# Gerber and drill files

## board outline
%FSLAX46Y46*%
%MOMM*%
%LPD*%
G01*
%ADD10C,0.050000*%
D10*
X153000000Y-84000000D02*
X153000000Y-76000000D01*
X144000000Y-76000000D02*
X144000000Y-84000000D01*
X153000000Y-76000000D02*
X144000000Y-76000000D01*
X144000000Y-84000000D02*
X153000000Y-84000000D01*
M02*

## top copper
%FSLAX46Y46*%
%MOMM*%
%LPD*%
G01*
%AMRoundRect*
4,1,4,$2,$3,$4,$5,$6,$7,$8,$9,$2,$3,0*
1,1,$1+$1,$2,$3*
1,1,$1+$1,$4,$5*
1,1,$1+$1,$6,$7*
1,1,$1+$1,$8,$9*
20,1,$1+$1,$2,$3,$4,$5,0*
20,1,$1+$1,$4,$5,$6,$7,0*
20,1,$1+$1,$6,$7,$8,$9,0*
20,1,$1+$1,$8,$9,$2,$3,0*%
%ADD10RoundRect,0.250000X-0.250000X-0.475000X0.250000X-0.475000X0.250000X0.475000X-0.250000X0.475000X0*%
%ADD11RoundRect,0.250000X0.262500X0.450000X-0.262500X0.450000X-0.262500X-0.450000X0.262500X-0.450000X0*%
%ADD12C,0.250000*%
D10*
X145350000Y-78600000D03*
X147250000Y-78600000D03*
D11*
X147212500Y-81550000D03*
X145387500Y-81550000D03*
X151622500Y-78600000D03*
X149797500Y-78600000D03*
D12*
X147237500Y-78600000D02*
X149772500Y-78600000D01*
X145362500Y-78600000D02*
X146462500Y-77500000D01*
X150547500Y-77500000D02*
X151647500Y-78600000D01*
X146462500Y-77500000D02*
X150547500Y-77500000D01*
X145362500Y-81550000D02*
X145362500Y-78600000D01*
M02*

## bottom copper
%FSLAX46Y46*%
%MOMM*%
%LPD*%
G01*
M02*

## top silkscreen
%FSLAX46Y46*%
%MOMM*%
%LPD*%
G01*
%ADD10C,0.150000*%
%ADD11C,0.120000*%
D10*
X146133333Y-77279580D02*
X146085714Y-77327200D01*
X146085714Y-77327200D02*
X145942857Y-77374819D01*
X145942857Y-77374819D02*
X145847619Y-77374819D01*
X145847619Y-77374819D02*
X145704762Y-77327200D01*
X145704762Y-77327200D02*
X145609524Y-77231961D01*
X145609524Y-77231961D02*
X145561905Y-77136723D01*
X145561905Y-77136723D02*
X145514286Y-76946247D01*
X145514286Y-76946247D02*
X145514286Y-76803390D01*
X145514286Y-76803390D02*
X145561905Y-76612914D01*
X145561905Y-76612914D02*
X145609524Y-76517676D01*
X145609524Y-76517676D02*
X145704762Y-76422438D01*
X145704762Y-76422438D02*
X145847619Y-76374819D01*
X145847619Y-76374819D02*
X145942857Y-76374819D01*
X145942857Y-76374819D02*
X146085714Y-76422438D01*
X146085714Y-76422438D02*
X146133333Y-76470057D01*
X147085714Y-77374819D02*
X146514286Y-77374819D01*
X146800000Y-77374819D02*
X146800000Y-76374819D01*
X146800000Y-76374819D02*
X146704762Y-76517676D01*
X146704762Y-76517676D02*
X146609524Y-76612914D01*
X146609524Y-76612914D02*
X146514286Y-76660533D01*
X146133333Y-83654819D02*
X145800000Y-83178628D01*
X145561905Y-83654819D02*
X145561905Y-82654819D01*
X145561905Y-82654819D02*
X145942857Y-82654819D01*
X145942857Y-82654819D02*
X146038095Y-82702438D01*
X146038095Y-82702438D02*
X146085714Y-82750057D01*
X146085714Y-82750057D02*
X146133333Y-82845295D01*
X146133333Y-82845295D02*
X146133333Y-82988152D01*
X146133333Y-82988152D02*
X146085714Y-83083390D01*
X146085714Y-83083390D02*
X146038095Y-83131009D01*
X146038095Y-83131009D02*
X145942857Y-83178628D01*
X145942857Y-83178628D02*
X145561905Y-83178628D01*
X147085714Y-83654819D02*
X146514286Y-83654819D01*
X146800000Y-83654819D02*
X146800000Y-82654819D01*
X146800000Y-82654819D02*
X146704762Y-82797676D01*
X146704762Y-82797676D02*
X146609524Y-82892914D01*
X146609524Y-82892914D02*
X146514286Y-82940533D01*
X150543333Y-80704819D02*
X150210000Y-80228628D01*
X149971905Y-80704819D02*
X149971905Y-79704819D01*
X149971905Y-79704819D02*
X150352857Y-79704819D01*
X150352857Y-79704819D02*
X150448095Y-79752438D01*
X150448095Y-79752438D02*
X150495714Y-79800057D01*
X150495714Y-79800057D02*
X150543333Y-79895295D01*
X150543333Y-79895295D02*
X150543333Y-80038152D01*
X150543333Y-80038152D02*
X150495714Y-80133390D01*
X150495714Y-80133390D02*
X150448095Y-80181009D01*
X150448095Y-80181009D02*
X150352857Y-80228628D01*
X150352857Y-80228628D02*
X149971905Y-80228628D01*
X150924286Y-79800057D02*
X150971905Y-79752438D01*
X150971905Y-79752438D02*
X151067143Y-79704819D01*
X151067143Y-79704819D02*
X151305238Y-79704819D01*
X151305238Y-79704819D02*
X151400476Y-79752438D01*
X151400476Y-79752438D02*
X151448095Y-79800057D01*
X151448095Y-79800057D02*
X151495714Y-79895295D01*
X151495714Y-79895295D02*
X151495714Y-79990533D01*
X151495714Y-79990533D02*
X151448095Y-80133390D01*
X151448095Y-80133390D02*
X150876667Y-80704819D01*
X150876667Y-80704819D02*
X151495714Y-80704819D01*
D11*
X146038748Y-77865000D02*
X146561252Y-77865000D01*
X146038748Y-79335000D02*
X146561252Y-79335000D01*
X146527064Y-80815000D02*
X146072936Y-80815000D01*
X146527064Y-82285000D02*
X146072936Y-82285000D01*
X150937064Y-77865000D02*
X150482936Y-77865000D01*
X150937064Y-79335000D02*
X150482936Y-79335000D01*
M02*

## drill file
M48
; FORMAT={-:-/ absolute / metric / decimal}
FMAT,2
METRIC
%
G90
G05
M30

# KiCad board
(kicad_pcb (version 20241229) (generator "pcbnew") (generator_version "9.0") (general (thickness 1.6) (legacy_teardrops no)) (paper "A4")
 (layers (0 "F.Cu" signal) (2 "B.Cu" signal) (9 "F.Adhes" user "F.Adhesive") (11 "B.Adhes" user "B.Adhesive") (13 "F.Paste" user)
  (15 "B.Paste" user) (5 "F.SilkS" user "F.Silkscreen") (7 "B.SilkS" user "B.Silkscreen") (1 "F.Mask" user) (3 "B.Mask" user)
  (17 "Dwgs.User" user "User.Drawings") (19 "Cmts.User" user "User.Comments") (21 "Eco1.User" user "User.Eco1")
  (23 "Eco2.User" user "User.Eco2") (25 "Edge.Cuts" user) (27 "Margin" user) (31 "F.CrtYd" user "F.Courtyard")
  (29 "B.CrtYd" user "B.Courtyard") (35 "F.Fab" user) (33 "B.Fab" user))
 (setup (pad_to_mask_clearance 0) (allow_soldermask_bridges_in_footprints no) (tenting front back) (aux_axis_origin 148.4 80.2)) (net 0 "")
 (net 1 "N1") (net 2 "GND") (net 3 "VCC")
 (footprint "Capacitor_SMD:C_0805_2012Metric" (layer "F.Cu") (at 146.3 78.6)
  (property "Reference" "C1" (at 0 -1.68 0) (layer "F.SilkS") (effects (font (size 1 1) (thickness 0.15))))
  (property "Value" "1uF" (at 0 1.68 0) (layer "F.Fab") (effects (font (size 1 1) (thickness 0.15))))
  (fp_line (start -0.261252 -0.735) (end 0.261252 -0.735) (stroke (width 0.12) (type solid)) (layer "F.SilkS"))
  (fp_line (start -0.261252 0.735) (end 0.261252 0.735) (stroke (width 0.12) (type solid)) (layer "F.SilkS"))
  (pad "1" smd roundrect (at -0.95 0) (size 1 1.45) (layers "F.Cu" "F.Mask" "F.Paste") (roundrect_rratio 0.25) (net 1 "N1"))
  (pad "2" smd roundrect (at 0.95 0) (size 1 1.45) (layers "F.Cu" "F.Mask" "F.Paste") (roundrect_rratio 0.25) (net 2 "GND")))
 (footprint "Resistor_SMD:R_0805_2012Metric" (layer "F.Cu") (at 146.3 81.55 180)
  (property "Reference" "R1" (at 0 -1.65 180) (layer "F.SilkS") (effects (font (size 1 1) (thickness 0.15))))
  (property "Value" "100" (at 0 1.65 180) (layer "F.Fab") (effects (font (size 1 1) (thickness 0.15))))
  (fp_line (start -0.227064 0.735) (end 0.227064 0.735) (stroke (width 0.12) (type solid)) (layer "F.SilkS"))
  (fp_line (start -0.227064 -0.735) (end 0.227064 -0.735) (stroke (width 0.12) (type solid)) (layer "F.SilkS"))
  (pad "1" smd roundrect (at -0.9125 0 180) (size 1.025 1.4) (layers "F.Cu" "F.Mask" "F.Paste") (roundrect_rratio 0.243902) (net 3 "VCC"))
  (pad "2" smd roundrect (at 0.9125 0 180) (size 1.025 1.4) (layers "F.Cu" "F.Mask" "F.Paste") (roundrect_rratio 0.243902) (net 1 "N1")))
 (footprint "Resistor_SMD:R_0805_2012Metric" (layer "F.Cu") (at 150.71 78.6 180)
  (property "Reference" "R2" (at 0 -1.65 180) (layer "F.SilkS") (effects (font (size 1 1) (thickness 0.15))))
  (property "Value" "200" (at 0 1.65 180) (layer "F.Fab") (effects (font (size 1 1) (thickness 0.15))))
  (fp_line (start -0.227064 0.735) (end 0.227064 0.735) (stroke (width 0.12) (type solid)) (layer "F.SilkS"))
  (fp_line (start -0.227064 -0.735) (end 0.227064 -0.735) (stroke (width 0.12) (type solid)) (layer "F.SilkS"))
  (pad "1" smd roundrect (at -0.9125 0 180) (size 1.025 1.4) (layers "F.Cu" "F.Mask" "F.Paste") (roundrect_rratio 0.243902) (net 1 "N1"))
  (pad "2" smd roundrect (at 0.9125 0 180) (size 1.025 1.4) (layers "F.Cu" "F.Mask" "F.Paste") (roundrect_rratio 0.243902) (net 2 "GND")))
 (gr_line (start 153 84) (end 153 76) (stroke (width 0.05) (type solid)) (layer "Edge.Cuts"))
 (gr_line (start 144 76) (end 144 84) (stroke (width 0.05) (type solid)) (layer "Edge.Cuts"))
 (gr_line (start 153 76) (end 144 76) (stroke (width 0.05) (type solid)) (layer "Edge.Cuts"))
 (gr_line (start 144 84) (end 153 84) (stroke (width 0.05) (type solid)) (layer "Edge.Cuts"))
 (segment (start 147.2375 78.6) (end 149.7725 78.6) (width 0.25) (layer "F.Cu") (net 2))
 (segment (start 145.3625 78.6) (end 146.4625 77.5) (width 0.25) (layer "F.Cu") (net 1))
 (segment (start 150.5475 77.5) (end 151.6475 78.6) (width 0.25) (layer "F.Cu") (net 1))
 (segment (start 146.4625 77.5) (end 150.5475 77.5) (width 0.25) (layer "F.Cu") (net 1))
 (segment (start 145.3625 81.55) (end 145.3625 78.6) (width 0.25) (layer "F.Cu") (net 1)))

